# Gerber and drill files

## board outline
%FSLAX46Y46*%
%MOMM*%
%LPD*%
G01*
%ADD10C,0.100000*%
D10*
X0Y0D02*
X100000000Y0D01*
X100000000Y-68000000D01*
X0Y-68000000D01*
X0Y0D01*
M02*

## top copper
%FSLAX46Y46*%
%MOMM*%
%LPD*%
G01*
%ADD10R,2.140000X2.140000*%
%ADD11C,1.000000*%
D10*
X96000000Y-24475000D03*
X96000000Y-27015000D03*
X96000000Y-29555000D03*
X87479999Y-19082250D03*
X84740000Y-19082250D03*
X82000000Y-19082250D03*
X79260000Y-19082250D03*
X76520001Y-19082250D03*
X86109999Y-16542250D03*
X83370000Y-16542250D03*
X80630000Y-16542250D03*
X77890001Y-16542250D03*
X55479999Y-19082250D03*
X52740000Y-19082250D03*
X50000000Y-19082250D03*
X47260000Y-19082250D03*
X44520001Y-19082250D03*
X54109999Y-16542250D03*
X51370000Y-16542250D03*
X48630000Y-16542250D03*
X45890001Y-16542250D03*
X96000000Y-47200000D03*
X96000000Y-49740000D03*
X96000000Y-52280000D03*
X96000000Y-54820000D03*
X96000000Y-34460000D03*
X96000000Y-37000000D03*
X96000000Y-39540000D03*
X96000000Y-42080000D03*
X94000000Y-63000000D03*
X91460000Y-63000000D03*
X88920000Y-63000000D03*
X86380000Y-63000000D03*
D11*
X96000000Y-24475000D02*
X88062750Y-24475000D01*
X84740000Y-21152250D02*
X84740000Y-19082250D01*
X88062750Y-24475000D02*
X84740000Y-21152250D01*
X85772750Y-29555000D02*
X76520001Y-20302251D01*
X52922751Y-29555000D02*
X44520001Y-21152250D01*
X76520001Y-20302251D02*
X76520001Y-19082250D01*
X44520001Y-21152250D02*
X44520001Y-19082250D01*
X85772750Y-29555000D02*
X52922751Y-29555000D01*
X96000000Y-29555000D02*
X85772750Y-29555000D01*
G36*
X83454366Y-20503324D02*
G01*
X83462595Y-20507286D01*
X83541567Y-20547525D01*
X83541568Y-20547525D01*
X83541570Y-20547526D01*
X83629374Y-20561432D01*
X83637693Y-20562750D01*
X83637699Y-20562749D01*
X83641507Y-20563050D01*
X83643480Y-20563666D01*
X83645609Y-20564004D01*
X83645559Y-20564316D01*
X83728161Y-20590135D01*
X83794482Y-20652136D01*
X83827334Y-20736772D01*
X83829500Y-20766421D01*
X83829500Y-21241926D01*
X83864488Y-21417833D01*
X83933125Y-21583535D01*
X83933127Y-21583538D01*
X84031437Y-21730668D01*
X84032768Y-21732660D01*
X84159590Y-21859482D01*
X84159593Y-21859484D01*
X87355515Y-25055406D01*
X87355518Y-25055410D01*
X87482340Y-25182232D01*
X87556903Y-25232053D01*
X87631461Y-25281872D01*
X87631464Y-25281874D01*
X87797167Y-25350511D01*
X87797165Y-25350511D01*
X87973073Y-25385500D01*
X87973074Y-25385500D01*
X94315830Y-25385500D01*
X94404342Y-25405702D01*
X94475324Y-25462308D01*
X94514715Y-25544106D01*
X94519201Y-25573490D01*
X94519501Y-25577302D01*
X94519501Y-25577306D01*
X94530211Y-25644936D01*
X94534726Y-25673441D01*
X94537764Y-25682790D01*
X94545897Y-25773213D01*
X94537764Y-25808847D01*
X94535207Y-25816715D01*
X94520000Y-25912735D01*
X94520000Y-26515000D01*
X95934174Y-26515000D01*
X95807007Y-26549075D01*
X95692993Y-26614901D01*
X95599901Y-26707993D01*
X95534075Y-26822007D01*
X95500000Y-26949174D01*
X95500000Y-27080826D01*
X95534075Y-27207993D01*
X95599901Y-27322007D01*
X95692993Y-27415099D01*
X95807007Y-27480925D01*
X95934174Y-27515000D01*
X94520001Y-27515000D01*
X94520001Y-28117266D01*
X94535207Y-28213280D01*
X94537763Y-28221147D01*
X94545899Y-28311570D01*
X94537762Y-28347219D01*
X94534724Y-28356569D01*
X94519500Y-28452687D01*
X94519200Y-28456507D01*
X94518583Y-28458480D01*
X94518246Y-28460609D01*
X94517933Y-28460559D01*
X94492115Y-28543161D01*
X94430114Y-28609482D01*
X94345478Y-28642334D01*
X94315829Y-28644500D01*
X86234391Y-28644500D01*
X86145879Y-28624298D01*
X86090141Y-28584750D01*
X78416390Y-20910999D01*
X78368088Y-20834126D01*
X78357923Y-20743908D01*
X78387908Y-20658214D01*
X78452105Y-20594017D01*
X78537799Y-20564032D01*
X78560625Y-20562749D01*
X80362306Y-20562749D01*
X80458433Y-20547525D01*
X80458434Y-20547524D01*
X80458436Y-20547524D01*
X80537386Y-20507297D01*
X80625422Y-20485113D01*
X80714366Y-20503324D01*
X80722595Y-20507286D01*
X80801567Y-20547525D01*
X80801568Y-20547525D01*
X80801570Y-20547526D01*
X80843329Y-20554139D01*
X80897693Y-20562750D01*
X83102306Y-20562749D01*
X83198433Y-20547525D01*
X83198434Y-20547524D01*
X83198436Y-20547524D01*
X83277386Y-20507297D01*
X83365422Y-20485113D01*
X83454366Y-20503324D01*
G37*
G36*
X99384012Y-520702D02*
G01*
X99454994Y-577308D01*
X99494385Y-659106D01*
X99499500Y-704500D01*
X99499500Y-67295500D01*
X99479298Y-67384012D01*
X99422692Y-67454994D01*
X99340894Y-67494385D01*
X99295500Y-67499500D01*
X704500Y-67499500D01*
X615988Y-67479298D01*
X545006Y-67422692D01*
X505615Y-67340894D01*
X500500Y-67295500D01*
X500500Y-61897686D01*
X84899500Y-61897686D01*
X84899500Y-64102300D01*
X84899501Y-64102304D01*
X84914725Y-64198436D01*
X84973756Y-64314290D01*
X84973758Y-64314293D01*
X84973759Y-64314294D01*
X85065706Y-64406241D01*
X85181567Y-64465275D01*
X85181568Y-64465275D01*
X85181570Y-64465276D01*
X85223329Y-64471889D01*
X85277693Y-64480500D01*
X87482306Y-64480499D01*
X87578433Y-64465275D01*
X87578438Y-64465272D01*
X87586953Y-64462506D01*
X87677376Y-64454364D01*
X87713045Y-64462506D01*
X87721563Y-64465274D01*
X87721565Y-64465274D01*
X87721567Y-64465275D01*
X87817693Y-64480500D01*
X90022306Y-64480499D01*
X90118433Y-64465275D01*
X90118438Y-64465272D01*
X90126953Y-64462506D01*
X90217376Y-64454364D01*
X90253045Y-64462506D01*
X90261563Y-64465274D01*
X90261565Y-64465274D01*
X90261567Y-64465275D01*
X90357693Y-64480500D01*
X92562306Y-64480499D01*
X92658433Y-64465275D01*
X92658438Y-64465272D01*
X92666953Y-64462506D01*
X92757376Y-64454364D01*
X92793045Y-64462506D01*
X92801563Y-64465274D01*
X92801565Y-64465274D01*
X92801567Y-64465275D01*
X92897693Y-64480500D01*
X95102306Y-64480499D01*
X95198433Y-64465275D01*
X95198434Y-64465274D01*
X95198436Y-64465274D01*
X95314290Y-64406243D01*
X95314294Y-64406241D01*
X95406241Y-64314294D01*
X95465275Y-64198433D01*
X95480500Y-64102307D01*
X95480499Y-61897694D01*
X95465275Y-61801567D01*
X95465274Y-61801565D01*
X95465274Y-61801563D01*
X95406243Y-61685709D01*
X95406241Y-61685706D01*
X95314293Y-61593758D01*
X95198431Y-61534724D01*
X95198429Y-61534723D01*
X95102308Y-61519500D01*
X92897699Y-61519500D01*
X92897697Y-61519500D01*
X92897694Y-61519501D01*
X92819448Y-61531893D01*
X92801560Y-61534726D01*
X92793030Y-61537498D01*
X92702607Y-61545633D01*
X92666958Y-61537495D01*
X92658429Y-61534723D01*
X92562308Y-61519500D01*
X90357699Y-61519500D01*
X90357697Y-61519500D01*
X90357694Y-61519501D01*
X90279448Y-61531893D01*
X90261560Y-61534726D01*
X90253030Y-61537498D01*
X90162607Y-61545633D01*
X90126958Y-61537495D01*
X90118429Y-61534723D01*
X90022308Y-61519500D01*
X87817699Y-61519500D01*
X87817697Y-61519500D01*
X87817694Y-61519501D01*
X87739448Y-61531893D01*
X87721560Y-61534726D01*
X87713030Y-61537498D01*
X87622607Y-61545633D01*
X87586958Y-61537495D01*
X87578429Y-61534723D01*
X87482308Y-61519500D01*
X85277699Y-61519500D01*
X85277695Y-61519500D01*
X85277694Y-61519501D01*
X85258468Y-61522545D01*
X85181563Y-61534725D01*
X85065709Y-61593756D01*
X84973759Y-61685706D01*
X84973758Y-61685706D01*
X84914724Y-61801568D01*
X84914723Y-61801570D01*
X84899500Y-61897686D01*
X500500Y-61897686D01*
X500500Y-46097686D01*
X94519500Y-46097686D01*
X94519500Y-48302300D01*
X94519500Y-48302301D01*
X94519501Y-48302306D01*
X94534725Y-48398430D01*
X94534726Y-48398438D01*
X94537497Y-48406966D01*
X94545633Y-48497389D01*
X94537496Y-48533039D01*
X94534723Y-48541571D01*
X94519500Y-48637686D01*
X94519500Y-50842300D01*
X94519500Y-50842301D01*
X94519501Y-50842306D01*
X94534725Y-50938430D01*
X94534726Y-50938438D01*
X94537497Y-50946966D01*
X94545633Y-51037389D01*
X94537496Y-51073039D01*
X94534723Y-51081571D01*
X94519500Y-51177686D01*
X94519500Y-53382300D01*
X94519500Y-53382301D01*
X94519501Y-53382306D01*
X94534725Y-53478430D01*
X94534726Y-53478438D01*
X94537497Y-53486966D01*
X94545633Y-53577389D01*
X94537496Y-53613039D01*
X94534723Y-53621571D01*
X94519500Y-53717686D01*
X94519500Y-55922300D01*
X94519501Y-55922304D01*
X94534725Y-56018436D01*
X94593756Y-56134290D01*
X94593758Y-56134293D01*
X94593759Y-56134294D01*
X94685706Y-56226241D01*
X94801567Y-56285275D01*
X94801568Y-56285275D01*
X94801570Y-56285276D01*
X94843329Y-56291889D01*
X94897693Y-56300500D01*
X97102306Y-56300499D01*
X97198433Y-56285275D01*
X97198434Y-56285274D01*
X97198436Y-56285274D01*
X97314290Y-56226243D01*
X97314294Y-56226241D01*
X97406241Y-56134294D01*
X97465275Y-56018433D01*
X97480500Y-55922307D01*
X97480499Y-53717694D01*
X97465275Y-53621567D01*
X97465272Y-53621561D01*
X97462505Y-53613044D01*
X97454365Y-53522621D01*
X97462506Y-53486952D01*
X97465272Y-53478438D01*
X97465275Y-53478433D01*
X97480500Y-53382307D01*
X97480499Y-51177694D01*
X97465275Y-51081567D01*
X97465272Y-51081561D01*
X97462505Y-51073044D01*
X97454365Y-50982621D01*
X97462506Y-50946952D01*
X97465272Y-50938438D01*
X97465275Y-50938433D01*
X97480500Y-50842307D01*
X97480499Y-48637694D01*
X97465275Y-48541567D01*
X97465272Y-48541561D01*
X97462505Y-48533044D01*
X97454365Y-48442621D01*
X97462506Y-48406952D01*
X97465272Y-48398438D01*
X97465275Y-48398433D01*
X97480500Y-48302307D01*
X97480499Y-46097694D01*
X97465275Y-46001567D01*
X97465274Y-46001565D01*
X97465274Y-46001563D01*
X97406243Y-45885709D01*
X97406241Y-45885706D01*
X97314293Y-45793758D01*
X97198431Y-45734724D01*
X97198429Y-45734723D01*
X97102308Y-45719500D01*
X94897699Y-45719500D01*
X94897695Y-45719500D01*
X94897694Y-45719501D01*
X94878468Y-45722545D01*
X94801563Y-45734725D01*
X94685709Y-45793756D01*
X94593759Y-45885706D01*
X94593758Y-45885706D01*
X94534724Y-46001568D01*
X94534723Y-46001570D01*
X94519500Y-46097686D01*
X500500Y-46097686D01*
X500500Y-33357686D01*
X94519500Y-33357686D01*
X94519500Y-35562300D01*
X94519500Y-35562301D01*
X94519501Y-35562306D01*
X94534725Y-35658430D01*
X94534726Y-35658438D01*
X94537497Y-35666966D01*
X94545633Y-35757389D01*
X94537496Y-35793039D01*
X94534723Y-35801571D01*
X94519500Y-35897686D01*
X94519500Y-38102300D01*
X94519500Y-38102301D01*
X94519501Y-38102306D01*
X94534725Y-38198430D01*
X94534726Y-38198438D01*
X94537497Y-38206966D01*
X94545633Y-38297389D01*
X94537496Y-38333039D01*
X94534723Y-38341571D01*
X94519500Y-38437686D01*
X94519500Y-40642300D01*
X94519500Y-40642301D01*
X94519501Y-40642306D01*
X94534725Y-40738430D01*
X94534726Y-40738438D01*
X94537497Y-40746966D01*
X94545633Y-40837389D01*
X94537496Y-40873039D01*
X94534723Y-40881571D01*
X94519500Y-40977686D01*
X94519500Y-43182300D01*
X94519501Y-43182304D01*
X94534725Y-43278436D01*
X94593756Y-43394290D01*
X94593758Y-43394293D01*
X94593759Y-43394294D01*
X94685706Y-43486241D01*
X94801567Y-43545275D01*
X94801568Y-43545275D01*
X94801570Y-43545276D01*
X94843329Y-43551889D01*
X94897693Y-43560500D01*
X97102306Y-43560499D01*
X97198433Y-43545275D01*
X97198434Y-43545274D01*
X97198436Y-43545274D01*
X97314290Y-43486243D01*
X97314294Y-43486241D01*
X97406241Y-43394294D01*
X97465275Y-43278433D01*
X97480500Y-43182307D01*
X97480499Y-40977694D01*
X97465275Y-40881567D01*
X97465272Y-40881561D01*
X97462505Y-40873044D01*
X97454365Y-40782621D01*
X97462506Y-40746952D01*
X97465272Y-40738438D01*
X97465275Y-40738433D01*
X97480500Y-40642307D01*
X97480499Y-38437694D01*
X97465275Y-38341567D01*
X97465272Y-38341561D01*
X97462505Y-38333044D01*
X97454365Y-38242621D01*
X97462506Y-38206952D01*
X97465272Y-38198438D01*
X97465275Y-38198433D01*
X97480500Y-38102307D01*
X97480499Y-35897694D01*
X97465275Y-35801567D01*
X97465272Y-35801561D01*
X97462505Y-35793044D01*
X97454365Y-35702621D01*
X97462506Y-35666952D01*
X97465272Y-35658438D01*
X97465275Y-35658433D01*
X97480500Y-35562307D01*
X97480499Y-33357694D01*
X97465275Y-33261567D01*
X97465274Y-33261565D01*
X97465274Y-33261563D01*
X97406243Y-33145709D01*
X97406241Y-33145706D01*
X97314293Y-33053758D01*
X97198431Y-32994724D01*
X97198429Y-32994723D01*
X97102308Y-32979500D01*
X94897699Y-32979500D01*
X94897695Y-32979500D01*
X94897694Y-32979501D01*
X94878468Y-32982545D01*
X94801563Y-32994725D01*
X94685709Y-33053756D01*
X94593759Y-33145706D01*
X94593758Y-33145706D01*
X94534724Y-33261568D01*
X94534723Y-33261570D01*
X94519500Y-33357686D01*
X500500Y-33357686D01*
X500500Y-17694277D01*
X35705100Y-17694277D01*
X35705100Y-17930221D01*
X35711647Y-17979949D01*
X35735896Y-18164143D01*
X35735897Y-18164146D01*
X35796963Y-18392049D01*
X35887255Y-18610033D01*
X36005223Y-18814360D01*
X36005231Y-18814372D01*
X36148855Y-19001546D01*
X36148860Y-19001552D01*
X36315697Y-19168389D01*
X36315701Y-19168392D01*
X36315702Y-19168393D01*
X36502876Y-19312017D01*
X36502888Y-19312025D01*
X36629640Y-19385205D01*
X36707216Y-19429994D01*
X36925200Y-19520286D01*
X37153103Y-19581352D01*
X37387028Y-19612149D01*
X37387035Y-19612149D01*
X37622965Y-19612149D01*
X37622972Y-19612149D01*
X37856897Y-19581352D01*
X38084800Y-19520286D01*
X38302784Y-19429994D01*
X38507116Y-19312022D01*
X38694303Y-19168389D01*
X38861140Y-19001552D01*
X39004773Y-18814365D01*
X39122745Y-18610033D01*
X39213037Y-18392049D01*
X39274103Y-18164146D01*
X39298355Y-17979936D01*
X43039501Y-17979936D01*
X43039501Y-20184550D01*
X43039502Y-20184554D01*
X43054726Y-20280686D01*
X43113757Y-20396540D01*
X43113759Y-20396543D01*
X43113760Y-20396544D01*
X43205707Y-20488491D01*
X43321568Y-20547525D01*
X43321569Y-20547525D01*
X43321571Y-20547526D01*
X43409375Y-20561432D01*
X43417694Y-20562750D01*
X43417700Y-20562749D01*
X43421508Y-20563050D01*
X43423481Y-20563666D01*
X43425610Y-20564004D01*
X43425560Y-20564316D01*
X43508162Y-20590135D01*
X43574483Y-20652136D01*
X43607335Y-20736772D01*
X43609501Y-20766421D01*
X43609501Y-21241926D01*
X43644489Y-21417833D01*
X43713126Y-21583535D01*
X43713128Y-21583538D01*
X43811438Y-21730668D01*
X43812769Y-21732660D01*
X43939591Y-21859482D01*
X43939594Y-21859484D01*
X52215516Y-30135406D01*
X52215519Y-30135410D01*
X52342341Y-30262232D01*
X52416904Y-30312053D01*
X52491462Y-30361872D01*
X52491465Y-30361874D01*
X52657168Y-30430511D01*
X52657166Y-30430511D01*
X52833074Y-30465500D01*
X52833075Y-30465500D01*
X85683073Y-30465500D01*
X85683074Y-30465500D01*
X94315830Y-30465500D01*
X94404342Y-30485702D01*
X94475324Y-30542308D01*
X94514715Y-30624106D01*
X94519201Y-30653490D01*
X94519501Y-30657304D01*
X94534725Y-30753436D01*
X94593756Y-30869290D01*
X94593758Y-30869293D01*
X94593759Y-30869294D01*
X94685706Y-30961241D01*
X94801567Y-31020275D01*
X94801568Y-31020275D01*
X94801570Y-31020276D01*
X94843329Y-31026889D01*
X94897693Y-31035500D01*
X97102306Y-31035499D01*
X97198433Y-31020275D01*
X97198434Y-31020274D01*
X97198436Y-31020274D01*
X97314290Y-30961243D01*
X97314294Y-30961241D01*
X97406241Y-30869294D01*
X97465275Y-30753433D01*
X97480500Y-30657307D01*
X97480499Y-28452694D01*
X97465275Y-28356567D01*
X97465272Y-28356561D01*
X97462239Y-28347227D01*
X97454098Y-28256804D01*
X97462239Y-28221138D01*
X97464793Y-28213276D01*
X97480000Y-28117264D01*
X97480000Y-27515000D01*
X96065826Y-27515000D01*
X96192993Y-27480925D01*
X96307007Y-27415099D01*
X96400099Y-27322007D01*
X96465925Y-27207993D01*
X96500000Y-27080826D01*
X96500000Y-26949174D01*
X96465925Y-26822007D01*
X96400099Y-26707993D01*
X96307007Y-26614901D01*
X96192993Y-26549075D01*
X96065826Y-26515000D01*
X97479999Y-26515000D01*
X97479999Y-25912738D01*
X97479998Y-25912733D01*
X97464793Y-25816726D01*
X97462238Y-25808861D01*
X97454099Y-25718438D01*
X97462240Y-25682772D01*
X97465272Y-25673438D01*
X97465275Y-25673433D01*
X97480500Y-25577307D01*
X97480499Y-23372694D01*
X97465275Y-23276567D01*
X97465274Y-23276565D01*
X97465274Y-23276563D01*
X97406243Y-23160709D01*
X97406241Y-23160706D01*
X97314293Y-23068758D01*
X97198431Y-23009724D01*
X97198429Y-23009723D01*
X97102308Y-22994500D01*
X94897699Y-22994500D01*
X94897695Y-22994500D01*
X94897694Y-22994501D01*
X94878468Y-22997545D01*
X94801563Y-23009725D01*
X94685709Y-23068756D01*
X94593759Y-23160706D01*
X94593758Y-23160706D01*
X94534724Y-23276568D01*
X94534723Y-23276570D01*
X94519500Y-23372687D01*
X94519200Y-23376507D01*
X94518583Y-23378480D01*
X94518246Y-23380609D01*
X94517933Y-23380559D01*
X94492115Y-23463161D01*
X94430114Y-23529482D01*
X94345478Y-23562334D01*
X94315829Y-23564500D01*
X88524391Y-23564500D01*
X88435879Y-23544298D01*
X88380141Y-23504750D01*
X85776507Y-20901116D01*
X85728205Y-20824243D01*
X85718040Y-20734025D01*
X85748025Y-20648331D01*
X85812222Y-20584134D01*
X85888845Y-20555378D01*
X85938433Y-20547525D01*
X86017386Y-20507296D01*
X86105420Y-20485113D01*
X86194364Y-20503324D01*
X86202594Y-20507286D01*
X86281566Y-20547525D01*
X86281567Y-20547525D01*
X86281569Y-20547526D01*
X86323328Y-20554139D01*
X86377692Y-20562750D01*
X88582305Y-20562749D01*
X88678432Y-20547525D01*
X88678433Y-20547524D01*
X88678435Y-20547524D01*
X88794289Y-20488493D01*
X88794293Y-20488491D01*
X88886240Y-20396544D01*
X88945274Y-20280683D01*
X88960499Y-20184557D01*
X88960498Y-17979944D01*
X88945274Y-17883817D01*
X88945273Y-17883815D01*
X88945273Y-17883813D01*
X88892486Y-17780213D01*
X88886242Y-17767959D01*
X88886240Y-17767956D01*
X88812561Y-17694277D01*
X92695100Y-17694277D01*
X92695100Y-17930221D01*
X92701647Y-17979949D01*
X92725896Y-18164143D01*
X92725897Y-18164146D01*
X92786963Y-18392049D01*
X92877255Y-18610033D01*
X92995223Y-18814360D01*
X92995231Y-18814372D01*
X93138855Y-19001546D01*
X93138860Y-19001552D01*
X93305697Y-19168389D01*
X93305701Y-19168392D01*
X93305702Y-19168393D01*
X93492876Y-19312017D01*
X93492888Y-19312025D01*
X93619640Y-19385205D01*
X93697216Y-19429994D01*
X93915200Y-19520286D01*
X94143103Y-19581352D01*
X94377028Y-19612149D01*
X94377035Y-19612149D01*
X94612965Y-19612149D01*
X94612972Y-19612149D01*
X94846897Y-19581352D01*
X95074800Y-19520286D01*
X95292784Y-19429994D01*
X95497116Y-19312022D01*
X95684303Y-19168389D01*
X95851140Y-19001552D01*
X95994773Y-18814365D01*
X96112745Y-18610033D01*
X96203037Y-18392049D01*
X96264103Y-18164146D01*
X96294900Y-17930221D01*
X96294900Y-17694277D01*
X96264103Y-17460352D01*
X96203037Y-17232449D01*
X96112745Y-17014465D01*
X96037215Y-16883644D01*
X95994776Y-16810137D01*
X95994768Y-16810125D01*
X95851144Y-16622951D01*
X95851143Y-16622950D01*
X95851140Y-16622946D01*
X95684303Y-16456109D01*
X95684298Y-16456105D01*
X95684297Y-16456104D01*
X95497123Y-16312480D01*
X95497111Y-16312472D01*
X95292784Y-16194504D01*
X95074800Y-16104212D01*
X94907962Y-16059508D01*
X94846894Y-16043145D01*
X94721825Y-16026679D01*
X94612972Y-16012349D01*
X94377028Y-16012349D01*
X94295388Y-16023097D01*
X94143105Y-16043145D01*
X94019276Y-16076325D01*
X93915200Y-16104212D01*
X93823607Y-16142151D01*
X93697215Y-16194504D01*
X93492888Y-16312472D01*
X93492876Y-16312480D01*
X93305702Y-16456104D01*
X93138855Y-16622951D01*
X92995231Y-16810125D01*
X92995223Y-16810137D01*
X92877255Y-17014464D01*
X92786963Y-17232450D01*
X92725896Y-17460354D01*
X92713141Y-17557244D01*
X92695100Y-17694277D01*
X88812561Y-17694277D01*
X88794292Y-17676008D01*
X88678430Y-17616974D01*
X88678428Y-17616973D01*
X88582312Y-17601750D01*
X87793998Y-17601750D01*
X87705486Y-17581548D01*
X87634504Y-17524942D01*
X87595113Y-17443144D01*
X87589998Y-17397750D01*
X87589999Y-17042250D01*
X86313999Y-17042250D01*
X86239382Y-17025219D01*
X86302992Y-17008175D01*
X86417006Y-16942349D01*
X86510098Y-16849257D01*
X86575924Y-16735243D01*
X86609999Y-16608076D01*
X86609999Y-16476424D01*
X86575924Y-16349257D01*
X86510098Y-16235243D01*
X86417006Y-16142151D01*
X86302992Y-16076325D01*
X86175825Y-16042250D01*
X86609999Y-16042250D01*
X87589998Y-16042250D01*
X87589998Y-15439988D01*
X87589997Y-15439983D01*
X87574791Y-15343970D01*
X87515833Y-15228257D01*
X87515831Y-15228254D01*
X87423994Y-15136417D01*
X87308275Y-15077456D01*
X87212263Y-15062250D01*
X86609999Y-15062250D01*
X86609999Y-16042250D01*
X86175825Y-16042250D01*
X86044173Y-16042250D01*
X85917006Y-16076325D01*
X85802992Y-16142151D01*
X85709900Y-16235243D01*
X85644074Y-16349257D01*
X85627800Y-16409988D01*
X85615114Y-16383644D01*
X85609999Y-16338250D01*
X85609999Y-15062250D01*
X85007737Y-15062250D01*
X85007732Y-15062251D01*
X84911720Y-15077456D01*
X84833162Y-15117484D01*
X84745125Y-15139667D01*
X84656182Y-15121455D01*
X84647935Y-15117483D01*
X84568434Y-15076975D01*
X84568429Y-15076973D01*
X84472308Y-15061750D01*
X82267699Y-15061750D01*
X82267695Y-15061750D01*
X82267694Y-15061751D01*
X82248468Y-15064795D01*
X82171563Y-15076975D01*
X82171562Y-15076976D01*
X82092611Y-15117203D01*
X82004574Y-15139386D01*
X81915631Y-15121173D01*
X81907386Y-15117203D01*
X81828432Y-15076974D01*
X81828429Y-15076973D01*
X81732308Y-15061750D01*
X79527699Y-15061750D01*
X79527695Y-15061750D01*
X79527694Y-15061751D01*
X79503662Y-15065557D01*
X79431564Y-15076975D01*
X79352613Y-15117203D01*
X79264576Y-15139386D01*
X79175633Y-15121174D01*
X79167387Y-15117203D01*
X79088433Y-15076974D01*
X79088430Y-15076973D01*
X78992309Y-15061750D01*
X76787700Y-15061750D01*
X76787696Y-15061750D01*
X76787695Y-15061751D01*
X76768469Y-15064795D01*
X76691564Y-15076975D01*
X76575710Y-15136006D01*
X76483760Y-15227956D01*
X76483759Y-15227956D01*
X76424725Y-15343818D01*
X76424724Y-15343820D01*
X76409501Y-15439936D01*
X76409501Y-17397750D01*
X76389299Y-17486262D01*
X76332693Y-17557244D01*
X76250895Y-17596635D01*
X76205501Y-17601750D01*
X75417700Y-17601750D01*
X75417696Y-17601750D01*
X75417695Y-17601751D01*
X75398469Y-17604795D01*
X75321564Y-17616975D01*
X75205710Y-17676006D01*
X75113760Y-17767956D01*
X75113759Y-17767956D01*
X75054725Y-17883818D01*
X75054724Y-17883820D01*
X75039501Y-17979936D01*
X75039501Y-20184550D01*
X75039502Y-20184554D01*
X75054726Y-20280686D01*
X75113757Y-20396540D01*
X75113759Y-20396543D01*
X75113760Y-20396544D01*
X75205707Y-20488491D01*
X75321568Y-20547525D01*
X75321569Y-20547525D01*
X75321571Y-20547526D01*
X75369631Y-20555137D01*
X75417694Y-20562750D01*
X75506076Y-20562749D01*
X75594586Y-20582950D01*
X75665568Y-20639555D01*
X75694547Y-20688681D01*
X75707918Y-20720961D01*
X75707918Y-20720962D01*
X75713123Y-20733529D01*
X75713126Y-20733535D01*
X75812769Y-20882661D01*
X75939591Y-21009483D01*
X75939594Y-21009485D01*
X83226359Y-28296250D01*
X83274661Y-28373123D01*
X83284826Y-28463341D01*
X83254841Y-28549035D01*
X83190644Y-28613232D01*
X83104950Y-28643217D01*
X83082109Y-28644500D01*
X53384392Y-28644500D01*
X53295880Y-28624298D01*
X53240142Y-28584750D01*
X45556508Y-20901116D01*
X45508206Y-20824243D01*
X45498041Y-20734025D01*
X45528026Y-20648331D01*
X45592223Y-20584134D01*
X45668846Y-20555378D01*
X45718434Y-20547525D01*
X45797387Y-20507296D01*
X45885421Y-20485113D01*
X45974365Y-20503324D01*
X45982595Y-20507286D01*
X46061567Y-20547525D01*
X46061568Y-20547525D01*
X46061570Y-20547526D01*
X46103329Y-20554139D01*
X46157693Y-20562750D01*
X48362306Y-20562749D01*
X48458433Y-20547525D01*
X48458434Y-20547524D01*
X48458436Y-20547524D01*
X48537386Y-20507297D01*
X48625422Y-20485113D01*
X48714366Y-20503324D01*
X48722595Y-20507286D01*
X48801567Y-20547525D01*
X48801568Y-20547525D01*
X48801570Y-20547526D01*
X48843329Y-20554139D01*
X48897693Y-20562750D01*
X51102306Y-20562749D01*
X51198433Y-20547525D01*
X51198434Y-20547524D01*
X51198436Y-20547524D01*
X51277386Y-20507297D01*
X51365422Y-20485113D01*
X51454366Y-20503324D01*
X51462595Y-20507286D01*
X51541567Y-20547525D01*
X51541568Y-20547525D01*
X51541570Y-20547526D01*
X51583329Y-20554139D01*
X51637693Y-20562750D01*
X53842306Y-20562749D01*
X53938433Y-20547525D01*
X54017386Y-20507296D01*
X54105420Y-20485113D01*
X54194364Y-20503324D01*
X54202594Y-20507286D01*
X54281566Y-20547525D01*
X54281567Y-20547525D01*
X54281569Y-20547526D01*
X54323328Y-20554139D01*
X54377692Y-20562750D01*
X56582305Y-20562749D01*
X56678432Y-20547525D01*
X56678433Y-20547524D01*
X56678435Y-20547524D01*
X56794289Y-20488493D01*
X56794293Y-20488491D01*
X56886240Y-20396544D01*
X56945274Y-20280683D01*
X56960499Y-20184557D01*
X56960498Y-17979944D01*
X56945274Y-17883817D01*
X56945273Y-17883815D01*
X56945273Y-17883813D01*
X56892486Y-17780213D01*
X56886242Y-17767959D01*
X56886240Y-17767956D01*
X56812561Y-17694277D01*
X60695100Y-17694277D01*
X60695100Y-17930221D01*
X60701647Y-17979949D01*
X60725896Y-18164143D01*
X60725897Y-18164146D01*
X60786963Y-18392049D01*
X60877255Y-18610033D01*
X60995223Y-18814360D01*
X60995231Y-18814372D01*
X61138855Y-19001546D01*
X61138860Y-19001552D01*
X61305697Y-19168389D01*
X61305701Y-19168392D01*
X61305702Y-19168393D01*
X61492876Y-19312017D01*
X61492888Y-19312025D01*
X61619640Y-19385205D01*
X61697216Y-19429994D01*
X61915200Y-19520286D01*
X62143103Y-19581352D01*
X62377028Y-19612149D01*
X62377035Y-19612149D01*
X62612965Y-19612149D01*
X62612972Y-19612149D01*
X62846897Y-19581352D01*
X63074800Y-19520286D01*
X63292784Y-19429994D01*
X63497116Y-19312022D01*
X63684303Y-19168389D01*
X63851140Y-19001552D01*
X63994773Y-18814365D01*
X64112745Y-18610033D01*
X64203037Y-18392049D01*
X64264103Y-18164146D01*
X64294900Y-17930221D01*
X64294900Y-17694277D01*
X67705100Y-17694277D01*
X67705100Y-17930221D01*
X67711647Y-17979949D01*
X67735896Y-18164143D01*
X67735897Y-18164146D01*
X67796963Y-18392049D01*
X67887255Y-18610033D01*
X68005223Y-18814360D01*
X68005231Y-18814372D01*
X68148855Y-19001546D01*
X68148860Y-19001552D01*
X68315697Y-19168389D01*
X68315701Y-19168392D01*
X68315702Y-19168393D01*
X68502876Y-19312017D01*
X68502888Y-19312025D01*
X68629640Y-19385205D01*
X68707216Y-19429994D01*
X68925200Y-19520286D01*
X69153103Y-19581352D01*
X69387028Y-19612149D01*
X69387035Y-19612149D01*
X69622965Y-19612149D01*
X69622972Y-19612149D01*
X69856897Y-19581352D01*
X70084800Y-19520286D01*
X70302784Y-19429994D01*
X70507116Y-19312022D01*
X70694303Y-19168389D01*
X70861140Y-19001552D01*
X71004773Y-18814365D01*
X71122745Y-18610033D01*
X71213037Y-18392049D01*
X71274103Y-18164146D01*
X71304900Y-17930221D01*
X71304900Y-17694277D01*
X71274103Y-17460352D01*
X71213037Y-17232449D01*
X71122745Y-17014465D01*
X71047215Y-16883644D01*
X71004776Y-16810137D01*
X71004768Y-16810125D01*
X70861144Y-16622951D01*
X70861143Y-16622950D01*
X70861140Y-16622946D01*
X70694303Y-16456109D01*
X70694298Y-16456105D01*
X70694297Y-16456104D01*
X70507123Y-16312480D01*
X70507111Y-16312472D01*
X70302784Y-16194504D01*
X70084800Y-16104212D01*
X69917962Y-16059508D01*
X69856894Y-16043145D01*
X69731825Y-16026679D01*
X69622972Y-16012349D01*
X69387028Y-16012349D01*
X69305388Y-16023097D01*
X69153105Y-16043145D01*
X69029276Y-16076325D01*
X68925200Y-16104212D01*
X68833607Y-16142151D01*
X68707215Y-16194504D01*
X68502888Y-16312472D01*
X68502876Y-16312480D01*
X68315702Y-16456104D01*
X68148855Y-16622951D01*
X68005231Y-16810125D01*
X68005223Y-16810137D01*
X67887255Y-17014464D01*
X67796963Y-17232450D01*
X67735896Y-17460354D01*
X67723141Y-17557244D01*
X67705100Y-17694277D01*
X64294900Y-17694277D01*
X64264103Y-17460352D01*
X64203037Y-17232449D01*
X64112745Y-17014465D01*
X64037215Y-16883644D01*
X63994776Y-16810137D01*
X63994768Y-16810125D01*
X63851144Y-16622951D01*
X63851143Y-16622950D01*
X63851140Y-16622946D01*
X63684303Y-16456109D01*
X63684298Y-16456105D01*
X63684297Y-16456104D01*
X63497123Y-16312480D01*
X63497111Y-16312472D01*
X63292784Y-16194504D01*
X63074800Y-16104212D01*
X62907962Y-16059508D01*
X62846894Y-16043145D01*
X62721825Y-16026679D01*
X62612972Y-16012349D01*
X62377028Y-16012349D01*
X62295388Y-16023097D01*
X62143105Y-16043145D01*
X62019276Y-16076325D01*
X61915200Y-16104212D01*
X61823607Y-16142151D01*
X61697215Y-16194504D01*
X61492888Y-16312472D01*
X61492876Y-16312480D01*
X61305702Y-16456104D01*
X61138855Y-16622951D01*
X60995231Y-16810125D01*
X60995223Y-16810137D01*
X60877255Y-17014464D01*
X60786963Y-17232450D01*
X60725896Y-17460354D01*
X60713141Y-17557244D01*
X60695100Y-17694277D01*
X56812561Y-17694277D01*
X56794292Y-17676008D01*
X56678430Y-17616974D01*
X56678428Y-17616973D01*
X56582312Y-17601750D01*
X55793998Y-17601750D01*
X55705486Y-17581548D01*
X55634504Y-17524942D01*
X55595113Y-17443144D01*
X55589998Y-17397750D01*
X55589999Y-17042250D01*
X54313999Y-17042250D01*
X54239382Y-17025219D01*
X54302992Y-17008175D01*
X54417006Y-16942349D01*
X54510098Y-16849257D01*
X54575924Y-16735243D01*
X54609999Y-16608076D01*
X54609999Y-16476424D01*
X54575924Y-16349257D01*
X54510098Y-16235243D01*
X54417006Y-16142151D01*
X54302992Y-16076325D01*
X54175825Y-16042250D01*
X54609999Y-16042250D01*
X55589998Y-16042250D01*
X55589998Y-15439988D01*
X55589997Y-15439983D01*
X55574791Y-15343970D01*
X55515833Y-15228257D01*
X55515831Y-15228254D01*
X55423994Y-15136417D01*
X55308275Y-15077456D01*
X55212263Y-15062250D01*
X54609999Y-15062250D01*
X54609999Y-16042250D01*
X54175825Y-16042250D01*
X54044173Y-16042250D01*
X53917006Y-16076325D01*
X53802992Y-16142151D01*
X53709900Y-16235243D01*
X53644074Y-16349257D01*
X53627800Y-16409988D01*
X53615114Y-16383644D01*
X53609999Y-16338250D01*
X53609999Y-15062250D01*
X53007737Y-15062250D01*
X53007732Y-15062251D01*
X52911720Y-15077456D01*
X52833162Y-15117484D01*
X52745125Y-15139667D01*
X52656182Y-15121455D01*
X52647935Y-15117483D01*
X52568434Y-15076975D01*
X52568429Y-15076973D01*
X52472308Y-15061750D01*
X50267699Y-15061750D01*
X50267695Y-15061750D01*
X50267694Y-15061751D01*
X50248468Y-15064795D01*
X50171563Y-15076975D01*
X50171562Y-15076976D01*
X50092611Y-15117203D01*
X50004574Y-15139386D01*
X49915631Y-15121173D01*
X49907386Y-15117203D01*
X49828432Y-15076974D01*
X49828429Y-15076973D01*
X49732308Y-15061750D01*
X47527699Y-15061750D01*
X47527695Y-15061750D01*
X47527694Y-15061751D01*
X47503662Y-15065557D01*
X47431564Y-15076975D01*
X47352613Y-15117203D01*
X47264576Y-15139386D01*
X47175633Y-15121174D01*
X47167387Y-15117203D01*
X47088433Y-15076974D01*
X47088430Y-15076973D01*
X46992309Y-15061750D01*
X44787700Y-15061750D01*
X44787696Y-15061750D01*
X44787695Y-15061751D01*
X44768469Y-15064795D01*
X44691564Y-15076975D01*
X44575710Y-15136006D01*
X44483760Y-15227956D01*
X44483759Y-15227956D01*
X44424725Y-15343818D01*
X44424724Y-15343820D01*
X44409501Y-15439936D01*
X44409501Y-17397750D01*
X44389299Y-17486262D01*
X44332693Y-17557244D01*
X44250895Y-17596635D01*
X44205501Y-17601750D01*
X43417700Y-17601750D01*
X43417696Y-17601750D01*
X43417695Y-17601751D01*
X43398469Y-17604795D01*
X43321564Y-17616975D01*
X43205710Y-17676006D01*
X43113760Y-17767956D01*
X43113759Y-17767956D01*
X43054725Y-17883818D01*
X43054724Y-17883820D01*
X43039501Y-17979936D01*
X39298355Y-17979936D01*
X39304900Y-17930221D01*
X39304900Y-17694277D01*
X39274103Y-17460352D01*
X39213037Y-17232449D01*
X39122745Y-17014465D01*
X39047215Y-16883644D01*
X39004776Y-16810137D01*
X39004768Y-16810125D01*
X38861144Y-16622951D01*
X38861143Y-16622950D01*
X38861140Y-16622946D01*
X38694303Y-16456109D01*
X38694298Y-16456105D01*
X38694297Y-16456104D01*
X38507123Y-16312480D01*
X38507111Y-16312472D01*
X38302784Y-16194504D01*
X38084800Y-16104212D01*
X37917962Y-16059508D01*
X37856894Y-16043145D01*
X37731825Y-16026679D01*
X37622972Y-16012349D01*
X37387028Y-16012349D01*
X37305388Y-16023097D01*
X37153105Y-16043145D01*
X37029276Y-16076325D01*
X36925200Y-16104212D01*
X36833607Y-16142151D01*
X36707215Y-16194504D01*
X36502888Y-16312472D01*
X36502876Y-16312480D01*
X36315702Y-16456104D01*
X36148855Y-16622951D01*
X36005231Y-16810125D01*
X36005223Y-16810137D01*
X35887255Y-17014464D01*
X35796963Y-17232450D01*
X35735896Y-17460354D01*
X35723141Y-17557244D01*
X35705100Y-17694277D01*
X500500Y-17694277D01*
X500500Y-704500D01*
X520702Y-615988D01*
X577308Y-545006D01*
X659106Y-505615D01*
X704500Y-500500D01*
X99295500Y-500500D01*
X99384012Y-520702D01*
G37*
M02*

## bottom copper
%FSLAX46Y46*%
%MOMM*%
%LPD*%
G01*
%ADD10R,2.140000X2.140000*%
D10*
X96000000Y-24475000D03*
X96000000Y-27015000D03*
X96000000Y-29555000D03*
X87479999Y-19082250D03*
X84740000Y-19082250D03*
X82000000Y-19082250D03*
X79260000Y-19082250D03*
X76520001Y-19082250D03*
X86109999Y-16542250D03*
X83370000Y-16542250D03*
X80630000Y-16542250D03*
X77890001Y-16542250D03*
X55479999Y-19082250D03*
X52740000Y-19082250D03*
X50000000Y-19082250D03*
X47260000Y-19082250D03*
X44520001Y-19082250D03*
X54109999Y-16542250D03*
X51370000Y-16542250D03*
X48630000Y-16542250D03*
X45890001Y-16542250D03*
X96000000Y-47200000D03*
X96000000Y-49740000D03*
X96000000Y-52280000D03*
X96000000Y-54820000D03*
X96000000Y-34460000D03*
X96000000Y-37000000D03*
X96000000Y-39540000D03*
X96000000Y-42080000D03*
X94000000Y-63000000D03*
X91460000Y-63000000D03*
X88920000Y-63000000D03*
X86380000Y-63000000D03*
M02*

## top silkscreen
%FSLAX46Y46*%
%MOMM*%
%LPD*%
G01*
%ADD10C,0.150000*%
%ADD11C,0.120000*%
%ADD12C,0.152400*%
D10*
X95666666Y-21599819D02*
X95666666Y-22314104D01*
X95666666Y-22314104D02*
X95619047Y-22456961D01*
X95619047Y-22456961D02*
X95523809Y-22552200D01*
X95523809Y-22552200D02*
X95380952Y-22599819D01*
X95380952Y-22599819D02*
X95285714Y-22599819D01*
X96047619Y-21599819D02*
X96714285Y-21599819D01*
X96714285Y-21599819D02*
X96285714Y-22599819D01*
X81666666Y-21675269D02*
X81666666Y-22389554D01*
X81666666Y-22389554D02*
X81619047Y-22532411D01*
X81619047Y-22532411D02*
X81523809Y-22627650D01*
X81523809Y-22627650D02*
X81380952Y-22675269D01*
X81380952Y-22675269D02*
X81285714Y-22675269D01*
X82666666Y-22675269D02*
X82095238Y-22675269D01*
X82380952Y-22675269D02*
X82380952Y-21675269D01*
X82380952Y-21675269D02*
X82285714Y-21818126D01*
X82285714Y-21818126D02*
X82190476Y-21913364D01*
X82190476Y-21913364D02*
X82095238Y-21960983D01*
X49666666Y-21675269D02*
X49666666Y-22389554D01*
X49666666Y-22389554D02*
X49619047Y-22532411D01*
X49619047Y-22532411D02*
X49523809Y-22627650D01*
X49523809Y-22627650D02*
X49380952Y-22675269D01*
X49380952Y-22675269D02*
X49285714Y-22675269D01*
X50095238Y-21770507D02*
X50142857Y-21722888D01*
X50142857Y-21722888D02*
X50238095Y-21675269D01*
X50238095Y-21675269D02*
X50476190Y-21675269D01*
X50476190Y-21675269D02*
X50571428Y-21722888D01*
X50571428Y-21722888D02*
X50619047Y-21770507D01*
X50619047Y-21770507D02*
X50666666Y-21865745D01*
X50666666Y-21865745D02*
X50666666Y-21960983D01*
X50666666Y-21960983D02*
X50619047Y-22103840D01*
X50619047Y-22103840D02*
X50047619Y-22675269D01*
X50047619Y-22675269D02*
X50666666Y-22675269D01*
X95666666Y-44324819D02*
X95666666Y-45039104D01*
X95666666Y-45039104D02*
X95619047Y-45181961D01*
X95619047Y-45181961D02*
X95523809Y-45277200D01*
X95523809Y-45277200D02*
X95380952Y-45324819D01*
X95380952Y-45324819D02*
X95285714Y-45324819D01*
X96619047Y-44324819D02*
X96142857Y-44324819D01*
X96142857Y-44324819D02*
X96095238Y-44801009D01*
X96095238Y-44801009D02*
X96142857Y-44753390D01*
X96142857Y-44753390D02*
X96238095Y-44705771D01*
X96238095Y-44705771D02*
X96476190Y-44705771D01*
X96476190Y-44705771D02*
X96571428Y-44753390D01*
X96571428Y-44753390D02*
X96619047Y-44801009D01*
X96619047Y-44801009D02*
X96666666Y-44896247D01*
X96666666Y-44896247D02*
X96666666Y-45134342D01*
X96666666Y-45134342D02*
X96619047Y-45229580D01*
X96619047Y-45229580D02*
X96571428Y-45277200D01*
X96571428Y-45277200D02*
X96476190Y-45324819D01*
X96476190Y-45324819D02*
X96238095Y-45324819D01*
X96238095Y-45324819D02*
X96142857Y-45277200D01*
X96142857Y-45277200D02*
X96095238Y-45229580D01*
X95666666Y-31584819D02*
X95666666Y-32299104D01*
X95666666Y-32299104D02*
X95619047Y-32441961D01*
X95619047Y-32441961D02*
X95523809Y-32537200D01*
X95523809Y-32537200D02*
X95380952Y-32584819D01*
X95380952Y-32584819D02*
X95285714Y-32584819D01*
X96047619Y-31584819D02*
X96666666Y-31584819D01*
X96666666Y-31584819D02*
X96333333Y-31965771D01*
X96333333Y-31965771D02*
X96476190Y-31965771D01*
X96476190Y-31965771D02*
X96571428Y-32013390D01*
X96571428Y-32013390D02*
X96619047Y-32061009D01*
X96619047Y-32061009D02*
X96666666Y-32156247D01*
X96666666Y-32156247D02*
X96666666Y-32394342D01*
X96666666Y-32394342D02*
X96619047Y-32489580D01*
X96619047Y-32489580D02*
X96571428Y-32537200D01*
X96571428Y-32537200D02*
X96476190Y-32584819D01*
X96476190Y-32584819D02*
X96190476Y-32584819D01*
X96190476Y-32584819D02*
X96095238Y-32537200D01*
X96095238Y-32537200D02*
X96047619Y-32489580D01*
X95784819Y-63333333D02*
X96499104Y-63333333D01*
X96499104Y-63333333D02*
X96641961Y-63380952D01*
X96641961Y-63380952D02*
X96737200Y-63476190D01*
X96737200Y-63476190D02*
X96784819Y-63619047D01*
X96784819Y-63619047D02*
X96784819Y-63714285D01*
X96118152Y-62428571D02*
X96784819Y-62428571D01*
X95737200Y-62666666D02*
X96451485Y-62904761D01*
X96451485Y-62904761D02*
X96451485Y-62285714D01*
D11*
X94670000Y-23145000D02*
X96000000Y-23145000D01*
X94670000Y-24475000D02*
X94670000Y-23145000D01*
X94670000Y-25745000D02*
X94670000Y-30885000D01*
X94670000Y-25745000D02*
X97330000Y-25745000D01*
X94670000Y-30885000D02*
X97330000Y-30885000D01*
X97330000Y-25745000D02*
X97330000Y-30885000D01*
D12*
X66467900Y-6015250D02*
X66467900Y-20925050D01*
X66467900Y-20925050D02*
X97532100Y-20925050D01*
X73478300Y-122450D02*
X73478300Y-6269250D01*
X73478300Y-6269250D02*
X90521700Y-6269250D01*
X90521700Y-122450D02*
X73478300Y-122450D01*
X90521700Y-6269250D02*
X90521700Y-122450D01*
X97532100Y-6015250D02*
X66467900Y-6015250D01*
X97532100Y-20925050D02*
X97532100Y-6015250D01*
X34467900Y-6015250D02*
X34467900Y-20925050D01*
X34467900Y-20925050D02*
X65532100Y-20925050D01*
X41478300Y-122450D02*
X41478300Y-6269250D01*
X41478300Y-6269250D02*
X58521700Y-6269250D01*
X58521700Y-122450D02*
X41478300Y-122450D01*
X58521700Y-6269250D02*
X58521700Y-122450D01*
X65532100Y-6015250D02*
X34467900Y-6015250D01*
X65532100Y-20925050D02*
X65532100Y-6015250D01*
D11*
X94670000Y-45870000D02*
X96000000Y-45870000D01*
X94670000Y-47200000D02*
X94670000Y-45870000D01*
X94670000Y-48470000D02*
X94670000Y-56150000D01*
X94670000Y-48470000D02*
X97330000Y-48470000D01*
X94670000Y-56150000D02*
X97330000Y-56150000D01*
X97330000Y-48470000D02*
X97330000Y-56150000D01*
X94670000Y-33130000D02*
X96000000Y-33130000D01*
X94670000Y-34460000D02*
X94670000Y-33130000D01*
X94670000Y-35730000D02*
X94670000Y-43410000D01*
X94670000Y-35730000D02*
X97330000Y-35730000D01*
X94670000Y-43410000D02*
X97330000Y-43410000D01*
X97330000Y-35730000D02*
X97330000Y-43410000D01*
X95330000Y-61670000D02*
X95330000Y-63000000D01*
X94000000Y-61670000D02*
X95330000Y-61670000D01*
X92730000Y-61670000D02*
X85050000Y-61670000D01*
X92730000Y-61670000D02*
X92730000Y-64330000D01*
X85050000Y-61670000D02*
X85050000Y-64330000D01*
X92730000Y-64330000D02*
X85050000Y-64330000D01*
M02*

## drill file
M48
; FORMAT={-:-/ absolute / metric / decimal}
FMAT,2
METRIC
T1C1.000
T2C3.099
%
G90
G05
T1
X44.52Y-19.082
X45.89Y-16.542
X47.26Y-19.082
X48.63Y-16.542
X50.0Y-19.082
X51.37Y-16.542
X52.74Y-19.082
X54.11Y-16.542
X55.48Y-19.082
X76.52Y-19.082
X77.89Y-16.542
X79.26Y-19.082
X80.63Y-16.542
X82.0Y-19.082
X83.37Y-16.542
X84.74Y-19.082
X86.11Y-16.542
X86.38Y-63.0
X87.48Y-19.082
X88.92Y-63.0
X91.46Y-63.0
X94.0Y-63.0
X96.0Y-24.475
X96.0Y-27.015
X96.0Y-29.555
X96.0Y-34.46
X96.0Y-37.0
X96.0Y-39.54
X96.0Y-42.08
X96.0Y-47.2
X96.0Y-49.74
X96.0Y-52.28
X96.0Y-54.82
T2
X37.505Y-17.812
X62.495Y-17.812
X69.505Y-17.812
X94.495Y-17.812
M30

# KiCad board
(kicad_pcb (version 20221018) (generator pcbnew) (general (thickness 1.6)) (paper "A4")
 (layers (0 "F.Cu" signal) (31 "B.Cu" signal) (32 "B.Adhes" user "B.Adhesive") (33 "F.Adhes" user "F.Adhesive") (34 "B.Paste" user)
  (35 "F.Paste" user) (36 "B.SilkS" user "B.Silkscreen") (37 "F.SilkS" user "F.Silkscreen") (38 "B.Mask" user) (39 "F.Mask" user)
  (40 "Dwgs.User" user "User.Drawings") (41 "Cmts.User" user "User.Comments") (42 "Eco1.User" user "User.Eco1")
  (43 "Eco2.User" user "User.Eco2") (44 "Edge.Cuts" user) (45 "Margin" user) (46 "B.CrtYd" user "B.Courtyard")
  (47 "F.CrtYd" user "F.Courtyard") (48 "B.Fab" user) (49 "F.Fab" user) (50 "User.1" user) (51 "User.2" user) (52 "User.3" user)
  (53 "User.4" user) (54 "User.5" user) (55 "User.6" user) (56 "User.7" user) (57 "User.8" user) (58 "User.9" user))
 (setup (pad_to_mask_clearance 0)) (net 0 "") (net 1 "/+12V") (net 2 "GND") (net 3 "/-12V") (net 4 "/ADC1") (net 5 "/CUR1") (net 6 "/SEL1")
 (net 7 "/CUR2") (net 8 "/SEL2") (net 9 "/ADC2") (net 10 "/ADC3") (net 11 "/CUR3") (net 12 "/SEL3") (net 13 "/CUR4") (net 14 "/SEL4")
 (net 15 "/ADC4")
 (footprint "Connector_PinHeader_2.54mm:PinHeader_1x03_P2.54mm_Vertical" (layer "F.Cu") (at 96 24.475)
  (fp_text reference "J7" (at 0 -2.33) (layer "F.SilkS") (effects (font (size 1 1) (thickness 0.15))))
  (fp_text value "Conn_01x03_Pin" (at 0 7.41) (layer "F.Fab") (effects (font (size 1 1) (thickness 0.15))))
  (fp_line (start -1.33 -1.33) (end 0 -1.33) (stroke (width 0.12) (type solid)) (layer "F.SilkS"))
  (fp_line (start -1.33 0) (end -1.33 -1.33) (stroke (width 0.12) (type solid)) (layer "F.SilkS"))
  (fp_line (start -1.33 1.27) (end -1.33 6.41) (stroke (width 0.12) (type solid)) (layer "F.SilkS"))
  (fp_line (start -1.33 1.27) (end 1.33 1.27) (stroke (width 0.12) (type solid)) (layer "F.SilkS"))
  (fp_line (start -1.33 6.41) (end 1.33 6.41) (stroke (width 0.12) (type solid)) (layer "F.SilkS"))
  (fp_line (start 1.33 1.27) (end 1.33 6.41) (stroke (width 0.12) (type solid)) (layer "F.SilkS"))
  (pad "1" thru_hole rect (at 0 0) (size 2.14 2.14) (drill 1) (layers "*.Cu" "*.Mask") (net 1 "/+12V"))
  (pad "2" thru_hole rect (at 0 2.54) (size 2.14 2.14) (drill 1) (layers "*.Cu" "*.Mask") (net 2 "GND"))
  (pad "3" thru_hole rect (at 0 5.08) (size 2.14 2.14) (drill 1) (layers "*.Cu" "*.Mask") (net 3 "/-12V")))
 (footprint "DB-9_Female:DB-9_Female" (layer "F.Cu") (at 82 6.14225)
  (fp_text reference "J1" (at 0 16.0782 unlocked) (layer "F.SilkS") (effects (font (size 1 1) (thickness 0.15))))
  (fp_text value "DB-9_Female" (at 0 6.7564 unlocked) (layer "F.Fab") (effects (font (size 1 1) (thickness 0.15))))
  (fp_line (start -15.5321 -0.127) (end -15.5321 14.7828) (stroke (width 0.1524) (type solid)) (layer "F.SilkS"))
  (fp_line (start -15.5321 14.7828) (end 15.5321 14.7828) (stroke (width 0.1524) (type solid)) (layer "F.SilkS"))
  (fp_line (start -8.5217 -6.0198) (end -8.5217 0.127) (stroke (width 0.1524) (type solid)) (layer "F.SilkS"))
  (fp_line (start -8.5217 0.127) (end 8.5217 0.127) (stroke (width 0.1524) (type solid)) (layer "F.SilkS"))
  (fp_line (start 8.5217 -6.0198) (end -8.5217 -6.0198) (stroke (width 0.1524) (type solid)) (layer "F.SilkS"))
  (fp_line (start 8.5217 0.127) (end 8.5217 -6.0198) (stroke (width 0.1524) (type solid)) (layer "F.SilkS"))
  (fp_line (start 15.5321 -0.127) (end -15.5321 -0.127) (stroke (width 0.1524) (type solid)) (layer "F.SilkS"))
  (fp_line (start 15.5321 14.7828) (end 15.5321 -0.127) (stroke (width 0.1524) (type solid)) (layer "F.SilkS"))
  (pad "" np_thru_hole circle (at -12.495 11.669999) (size 3.0988 3.0988) (drill 3.0988) (layers "*.Cu" "*.Mask"))
  (pad "" np_thru_hole circle (at 12.495 11.669999) (size 3.0988 3.0988) (drill 3.0988) (layers "*.Cu" "*.Mask"))
  (pad "1" thru_hole rect (at 5.479999 12.94) (size 2.14 2.14) (drill 1) (layers "*.Cu" "*.Mask") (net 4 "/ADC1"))
  (pad "2" thru_hole rect (at 2.74 12.94) (size 2.14 2.14) (drill 1) (layers "*.Cu" "*.Mask") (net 1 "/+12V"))
  (pad "3" thru_hole rect (at 0 12.94) (size 2.14 2.14) (drill 1) (layers "*.Cu" "*.Mask") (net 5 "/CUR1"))
  (pad "4" thru_hole rect (at -2.74 12.94) (size 2.14 2.14) (drill 1) (layers "*.Cu" "*.Mask") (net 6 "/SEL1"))
  (pad "5" thru_hole rect (at -5.479999 12.94) (size 2.14 2.14) (drill 1) (layers "*.Cu" "*.Mask") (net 3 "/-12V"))
  (pad "6" thru_hole rect (at 4.109999 10.4) (size 2.14 2.14) (drill 1) (layers "*.Cu" "*.Mask") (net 2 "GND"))
  (pad "7" thru_hole rect (at 1.37 10.4) (size 2.14 2.14) (drill 1) (layers "*.Cu" "*.Mask") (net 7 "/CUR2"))
  (pad "8" thru_hole rect (at -1.37 10.4) (size 2.14 2.14) (drill 1) (layers "*.Cu" "*.Mask") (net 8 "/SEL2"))
  (pad "9" thru_hole rect (at -4.109999 10.4) (size 2.14 2.14) (drill 1) (layers "*.Cu" "*.Mask") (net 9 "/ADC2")))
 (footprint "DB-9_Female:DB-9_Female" (layer "F.Cu") (at 50 6.14225)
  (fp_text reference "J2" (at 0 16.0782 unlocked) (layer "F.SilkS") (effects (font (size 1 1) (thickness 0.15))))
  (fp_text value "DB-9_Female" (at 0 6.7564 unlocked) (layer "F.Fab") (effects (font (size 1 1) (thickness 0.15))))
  (fp_line (start -15.5321 -0.127) (end -15.5321 14.7828) (stroke (width 0.1524) (type solid)) (layer "F.SilkS"))
  (fp_line (start -15.5321 14.7828) (end 15.5321 14.7828) (stroke (width 0.1524) (type solid)) (layer "F.SilkS"))
  (fp_line (start -8.5217 -6.0198) (end -8.5217 0.127) (stroke (width 0.1524) (type solid)) (layer "F.SilkS"))
  (fp_line (start -8.5217 0.127) (end 8.5217 0.127) (stroke (width 0.1524) (type solid)) (layer "F.SilkS"))
  (fp_line (start 8.5217 -6.0198) (end -8.5217 -6.0198) (stroke (width 0.1524) (type solid)) (layer "F.SilkS"))
  (fp_line (start 8.5217 0.127) (end 8.5217 -6.0198) (stroke (width 0.1524) (type solid)) (layer "F.SilkS"))
  (fp_line (start 15.5321 -0.127) (end -15.5321 -0.127) (stroke (width 0.1524) (type solid)) (layer "F.SilkS"))
  (fp_line (start 15.5321 14.7828) (end 15.5321 -0.127) (stroke (width 0.1524) (type solid)) (layer "F.SilkS"))
  (pad "" np_thru_hole circle (at -12.495 11.669999) (size 3.0988 3.0988) (drill 3.0988) (layers "*.Cu" "*.Mask"))
  (pad "" np_thru_hole circle (at 12.495 11.669999) (size 3.0988 3.0988) (drill 3.0988) (layers "*.Cu" "*.Mask"))
  (pad "1" thru_hole rect (at 5.479999 12.94) (size 2.14 2.14) (drill 1) (layers "*.Cu" "*.Mask") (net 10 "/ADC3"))
  (pad "2" thru_hole rect (at 2.74 12.94) (size 2.14 2.14) (drill 1) (layers "*.Cu" "*.Mask") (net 1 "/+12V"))
  (pad "3" thru_hole rect (at 0 12.94) (size 2.14 2.14) (drill 1) (layers "*.Cu" "*.Mask") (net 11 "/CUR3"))
  (pad "4" thru_hole rect (at -2.74 12.94) (size 2.14 2.14) (drill 1) (layers "*.Cu" "*.Mask") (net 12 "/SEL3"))
  (pad "5" thru_hole rect (at -5.479999 12.94) (size 2.14 2.14) (drill 1) (layers "*.Cu" "*.Mask") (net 3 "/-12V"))
  (pad "6" thru_hole rect (at 4.109999 10.4) (size 2.14 2.14) (drill 1) (layers "*.Cu" "*.Mask") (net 2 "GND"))
  (pad "7" thru_hole rect (at 1.37 10.4) (size 2.14 2.14) (drill 1) (layers "*.Cu" "*.Mask") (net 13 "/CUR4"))
  (pad "8" thru_hole rect (at -1.37 10.4) (size 2.14 2.14) (drill 1) (layers "*.Cu" "*.Mask") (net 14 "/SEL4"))
  (pad "9" thru_hole rect (at -4.109999 10.4) (size 2.14 2.14) (drill 1) (layers "*.Cu" "*.Mask") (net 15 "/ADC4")))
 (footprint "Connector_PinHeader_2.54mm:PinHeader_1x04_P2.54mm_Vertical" (layer "F.Cu") (at 96 47.2)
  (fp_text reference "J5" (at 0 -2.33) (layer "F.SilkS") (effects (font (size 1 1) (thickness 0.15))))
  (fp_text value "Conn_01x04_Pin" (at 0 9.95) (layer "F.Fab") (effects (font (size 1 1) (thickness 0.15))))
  (fp_line (start -1.33 -1.33) (end 0 -1.33) (stroke (width 0.12) (type solid)) (layer "F.SilkS"))
  (fp_line (start -1.33 0) (end -1.33 -1.33) (stroke (width 0.12) (type solid)) (layer "F.SilkS"))
  (fp_line (start -1.33 1.27) (end -1.33 8.95) (stroke (width 0.12) (type solid)) (layer "F.SilkS"))
  (fp_line (start -1.33 1.27) (end 1.33 1.27) (stroke (width 0.12) (type solid)) (layer "F.SilkS"))
  (fp_line (start -1.33 8.95) (end 1.33 8.95) (stroke (width 0.12) (type solid)) (layer "F.SilkS"))
  (fp_line (start 1.33 1.27) (end 1.33 8.95) (stroke (width 0.12) (type solid)) (layer "F.SilkS"))
  (pad "1" thru_hole rect (at 0 0) (size 2.14 2.14) (drill 1) (layers "*.Cu" "*.Mask") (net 5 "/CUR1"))
  (pad "2" thru_hole rect (at 0 2.54) (size 2.14 2.14) (drill 1) (layers "*.Cu" "*.Mask") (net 7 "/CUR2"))
  (pad "3" thru_hole rect (at 0 5.08) (size 2.14 2.14) (drill 1) (layers "*.Cu" "*.Mask") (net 11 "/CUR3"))
  (pad "4" thru_hole rect (at 0 7.62) (size 2.14 2.14) (drill 1) (layers "*.Cu" "*.Mask") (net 13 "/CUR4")))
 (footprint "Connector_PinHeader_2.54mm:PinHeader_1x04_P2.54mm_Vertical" (layer "F.Cu") (at 96 34.46)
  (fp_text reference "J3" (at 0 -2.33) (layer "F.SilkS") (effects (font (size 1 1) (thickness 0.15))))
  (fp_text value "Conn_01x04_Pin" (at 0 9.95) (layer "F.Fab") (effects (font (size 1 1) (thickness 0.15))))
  (fp_line (start -1.33 -1.33) (end 0 -1.33) (stroke (width 0.12) (type solid)) (layer "F.SilkS"))
  (fp_line (start -1.33 0) (end -1.33 -1.33) (stroke (width 0.12) (type solid)) (layer "F.SilkS"))
  (fp_line (start -1.33 1.27) (end -1.33 8.95) (stroke (width 0.12) (type solid)) (layer "F.SilkS"))
  (fp_line (start -1.33 1.27) (end 1.33 1.27) (stroke (width 0.12) (type solid)) (layer "F.SilkS"))
  (fp_line (start -1.33 8.95) (end 1.33 8.95) (stroke (width 0.12) (type solid)) (layer "F.SilkS"))
  (fp_line (start 1.33 1.27) (end 1.33 8.95) (stroke (width 0.12) (type solid)) (layer "F.SilkS"))
  (pad "1" thru_hole rect (at 0 0) (size 2.14 2.14) (drill 1) (layers "*.Cu" "*.Mask") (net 4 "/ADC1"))
  (pad "2" thru_hole rect (at 0 2.54) (size 2.14 2.14) (drill 1) (layers "*.Cu" "*.Mask") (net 9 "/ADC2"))
  (pad "3" thru_hole rect (at 0 5.08) (size 2.14 2.14) (drill 1) (layers "*.Cu" "*.Mask") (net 10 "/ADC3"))
  (pad "4" thru_hole rect (at 0 7.62) (size 2.14 2.14) (drill 1) (layers "*.Cu" "*.Mask") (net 15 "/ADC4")))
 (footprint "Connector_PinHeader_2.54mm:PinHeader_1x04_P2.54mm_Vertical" (layer "F.Cu") (at 94 63 -90)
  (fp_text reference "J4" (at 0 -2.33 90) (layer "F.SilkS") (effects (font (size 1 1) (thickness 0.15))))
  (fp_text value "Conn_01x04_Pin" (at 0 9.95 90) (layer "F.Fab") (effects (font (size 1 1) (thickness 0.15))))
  (fp_line (start -1.33 -1.33) (end 0 -1.33) (stroke (width 0.12) (type solid)) (layer "F.SilkS"))
  (fp_line (start -1.33 0) (end -1.33 -1.33) (stroke (width 0.12) (type solid)) (layer "F.SilkS"))
  (fp_line (start -1.33 1.27) (end -1.33 8.95) (stroke (width 0.12) (type solid)) (layer "F.SilkS"))
  (fp_line (start -1.33 1.27) (end 1.33 1.27) (stroke (width 0.12) (type solid)) (layer "F.SilkS"))
  (fp_line (start -1.33 8.95) (end 1.33 8.95) (stroke (width 0.12) (type solid)) (layer "F.SilkS"))
  (fp_line (start 1.33 1.27) (end 1.33 8.95) (stroke (width 0.12) (type solid)) (layer "F.SilkS"))
  (pad "1" thru_hole rect (at 0 0 270) (size 2.14 2.14) (drill 1) (layers "*.Cu" "*.Mask") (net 6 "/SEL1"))
  (pad "2" thru_hole rect (at 0 2.54 270) (size 2.14 2.14) (drill 1) (layers "*.Cu" "*.Mask") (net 8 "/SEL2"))
  (pad "3" thru_hole rect (at 0 5.08 270) (size 2.14 2.14) (drill 1) (layers "*.Cu" "*.Mask") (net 12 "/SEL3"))
  (pad "4" thru_hole rect (at 0 7.62 270) (size 2.14 2.14) (drill 1) (layers "*.Cu" "*.Mask") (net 14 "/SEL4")))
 (gr_rect (start 0 0) (end 100 68) (stroke (width 0.1) (type default)) (fill none) (layer "Edge.Cuts"))
 (segment (start 96 24.475) (end 88.06275 24.475) (width 1) (layer "F.Cu") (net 1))
 (segment (start 84.74 21.15225) (end 84.74 19.08225) (width 1) (layer "F.Cu") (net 1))
 (segment (start 88.06275 24.475) (end 84.74 21.15225) (width 1) (layer "F.Cu") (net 1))
 (segment (start 85.77275 29.555) (end 76.520001 20.302251) (width 1) (layer "F.Cu") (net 3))
 (segment (start 52.922751 29.555) (end 44.520001 21.15225) (width 1) (layer "F.Cu") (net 3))
 (segment (start 76.520001 20.302251) (end 76.520001 19.08225) (width 1) (layer "F.Cu") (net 3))
 (segment (start 44.520001 21.15225) (end 44.520001 19.08225) (width 1) (layer "F.Cu") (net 3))
 (segment (start 85.77275 29.555) (end 52.922751 29.555) (width 1) (layer "F.Cu") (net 3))
 (segment (start 96 29.555) (end 85.77275 29.555) (width 1) (layer "F.Cu") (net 3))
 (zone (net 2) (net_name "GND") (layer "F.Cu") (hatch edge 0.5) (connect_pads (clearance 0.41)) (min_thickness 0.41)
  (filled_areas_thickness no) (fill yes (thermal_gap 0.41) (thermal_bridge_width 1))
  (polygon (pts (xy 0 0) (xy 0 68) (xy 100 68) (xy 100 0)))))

